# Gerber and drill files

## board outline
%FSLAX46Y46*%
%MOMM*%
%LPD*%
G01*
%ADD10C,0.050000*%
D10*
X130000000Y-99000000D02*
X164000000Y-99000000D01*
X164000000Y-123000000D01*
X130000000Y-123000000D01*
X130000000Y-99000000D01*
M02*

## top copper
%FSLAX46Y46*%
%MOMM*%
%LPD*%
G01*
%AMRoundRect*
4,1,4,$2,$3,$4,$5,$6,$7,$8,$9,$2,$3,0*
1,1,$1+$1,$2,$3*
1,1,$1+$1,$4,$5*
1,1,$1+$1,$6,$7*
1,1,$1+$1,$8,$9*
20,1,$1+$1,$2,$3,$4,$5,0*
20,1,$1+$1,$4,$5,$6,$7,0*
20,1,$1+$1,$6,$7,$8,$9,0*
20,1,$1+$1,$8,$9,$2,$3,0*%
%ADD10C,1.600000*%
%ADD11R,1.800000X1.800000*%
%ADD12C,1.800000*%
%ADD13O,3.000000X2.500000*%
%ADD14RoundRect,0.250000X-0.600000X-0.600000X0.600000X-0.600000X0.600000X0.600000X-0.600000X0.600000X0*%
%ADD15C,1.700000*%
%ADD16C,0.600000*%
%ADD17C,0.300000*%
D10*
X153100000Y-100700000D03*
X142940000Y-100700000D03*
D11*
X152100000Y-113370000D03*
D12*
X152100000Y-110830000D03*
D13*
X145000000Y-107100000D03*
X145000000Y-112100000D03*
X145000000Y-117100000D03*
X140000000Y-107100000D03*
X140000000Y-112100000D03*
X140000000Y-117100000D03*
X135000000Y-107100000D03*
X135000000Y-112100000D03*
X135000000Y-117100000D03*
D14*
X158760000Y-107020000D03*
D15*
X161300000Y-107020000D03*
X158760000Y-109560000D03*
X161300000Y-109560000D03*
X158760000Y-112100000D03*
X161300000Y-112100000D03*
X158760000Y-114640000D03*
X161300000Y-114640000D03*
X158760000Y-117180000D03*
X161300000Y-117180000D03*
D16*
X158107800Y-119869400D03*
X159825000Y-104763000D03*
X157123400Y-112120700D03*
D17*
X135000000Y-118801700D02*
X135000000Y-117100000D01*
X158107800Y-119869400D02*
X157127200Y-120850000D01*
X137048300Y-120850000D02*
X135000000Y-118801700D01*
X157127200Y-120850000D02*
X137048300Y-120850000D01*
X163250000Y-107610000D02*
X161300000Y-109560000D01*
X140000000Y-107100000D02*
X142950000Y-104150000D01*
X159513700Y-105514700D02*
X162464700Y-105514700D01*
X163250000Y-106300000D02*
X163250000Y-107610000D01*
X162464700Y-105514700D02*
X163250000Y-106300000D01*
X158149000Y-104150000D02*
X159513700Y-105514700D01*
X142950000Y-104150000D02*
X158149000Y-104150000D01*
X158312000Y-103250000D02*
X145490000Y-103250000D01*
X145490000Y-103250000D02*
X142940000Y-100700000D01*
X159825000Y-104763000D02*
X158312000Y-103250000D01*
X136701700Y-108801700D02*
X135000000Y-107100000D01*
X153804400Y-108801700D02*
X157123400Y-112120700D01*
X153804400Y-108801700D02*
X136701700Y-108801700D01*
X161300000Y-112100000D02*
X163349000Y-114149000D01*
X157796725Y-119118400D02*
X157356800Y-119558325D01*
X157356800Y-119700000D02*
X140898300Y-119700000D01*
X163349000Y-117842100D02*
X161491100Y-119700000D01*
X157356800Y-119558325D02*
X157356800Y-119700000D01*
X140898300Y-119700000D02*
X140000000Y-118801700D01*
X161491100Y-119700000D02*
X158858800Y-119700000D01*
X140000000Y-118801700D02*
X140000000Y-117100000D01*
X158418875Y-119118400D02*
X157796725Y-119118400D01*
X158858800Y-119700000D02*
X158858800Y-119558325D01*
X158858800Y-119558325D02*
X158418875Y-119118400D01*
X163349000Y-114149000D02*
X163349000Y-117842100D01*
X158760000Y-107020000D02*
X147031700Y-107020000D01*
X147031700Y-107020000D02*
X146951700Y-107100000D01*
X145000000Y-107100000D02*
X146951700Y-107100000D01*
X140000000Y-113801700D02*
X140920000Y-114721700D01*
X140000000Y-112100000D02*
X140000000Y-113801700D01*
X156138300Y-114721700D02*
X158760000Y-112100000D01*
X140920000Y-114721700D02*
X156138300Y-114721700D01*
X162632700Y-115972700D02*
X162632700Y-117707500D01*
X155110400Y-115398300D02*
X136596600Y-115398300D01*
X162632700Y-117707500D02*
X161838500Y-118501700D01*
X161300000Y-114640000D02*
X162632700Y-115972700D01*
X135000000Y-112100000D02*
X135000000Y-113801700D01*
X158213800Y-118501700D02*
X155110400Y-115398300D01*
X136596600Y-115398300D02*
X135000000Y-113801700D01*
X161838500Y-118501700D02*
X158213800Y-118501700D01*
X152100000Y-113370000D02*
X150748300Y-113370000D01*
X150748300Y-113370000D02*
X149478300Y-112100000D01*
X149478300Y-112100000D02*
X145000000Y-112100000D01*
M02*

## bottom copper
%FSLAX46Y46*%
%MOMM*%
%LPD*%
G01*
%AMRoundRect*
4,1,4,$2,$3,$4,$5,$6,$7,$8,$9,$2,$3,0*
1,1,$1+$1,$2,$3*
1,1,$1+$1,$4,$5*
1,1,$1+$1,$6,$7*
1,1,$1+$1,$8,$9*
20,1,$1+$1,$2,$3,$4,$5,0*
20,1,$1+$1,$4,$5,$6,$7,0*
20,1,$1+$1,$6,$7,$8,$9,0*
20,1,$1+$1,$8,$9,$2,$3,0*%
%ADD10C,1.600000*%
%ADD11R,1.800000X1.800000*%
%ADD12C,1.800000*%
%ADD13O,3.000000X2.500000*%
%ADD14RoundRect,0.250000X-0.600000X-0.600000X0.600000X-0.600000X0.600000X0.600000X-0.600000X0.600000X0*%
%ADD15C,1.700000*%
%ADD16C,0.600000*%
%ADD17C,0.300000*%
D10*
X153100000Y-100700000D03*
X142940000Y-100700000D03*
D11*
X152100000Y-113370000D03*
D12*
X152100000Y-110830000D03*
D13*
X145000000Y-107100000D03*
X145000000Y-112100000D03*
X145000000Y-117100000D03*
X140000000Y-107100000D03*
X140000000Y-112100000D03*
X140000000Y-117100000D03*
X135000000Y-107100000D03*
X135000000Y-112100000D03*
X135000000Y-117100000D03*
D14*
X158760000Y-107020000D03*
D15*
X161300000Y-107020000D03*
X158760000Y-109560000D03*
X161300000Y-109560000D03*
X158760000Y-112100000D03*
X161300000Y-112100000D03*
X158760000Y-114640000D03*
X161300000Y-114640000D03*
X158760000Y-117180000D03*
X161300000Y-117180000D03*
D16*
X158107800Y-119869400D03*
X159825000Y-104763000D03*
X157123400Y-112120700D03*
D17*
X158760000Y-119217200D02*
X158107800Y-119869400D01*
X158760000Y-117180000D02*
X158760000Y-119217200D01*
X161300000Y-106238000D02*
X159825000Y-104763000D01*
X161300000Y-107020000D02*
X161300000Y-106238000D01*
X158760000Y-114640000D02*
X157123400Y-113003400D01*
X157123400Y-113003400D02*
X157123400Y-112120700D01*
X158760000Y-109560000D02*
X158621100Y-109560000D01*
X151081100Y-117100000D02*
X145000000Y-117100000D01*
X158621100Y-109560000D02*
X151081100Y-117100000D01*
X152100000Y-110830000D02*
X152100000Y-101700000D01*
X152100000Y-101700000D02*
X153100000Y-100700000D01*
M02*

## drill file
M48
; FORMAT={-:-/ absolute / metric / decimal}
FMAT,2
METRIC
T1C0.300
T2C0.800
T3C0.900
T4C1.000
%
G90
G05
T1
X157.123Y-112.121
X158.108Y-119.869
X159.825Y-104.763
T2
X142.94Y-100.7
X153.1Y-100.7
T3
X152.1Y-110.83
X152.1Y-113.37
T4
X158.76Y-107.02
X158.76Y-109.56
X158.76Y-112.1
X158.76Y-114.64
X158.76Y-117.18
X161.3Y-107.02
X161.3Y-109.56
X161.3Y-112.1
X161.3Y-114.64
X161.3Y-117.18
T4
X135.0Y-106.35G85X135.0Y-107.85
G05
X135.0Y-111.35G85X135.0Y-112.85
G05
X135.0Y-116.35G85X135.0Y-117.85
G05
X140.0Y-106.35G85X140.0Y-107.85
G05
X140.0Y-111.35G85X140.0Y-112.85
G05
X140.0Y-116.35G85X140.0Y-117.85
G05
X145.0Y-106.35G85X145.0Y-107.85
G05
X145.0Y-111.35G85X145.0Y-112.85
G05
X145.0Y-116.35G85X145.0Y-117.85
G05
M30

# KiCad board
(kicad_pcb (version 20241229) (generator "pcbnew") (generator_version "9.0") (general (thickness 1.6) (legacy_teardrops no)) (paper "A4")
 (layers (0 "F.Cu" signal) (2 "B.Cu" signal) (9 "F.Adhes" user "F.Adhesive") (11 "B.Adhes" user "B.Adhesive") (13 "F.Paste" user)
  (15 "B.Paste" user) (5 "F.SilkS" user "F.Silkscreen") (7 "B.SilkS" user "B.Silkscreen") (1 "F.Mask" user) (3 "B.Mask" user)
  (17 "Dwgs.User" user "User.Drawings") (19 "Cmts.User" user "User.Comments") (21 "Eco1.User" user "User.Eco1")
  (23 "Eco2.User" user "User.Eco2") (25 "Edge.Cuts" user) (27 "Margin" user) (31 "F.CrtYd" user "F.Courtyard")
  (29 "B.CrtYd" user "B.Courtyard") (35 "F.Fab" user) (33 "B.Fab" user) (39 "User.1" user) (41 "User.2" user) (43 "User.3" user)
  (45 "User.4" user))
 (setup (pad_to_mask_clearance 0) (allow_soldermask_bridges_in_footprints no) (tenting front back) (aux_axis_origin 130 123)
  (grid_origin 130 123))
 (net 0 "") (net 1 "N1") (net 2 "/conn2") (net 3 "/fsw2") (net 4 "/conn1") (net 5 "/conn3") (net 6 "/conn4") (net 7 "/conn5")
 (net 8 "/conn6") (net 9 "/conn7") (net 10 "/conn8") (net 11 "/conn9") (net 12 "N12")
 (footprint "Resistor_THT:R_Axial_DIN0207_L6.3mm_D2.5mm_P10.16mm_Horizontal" (layer "F.Cu") (at 153.1 100.7 180)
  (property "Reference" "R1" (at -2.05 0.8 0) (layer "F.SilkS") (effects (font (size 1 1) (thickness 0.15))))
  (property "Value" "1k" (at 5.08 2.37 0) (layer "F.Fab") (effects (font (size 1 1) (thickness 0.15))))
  (pad "1" thru_hole circle (at 0 0 180) (size 1.6 1.6) (drill 0.8) (layers "*.Cu" "*.Mask") (remove_unused_layers no) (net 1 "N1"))
  (pad "2" thru_hole circle (at 10.16 0 180) (size 1.6 1.6) (drill 0.8) (layers "*.Cu" "*.Mask") (remove_unused_layers no) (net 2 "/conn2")))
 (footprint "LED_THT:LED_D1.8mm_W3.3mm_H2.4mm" (layer "F.Cu") (at 152.1 113.37 90)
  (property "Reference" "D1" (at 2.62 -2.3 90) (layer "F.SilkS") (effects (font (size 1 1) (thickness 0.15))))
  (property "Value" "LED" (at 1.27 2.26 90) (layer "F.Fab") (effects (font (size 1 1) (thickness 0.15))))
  (pad "1" thru_hole rect (at 0 0 90) (size 1.8 1.8) (drill 0.9) (layers "*.Cu" "*.Mask") (remove_unused_layers no) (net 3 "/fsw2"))
  (pad "2" thru_hole circle (at 2.54 0 90) (size 1.8 1.8) (drill 0.9) (layers "*.Cu" "*.Mask") (remove_unused_layers no) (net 1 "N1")))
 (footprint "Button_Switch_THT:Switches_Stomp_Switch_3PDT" (layer "F.Cu") (at 140 112.1 -90)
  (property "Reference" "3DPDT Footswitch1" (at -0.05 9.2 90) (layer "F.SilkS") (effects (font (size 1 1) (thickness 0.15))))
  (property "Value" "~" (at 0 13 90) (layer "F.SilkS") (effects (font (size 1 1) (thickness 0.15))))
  (pad "1" thru_hole oval (at -5 -5 270) (size 2.5 3) (drill oval 2.5 1) (layers "*.Cu" "*.Mask" "F.SilkS") (remove_unused_layers no)
   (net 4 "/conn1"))
  (pad "2" thru_hole oval (at 0 -5 270) (size 2.5 3) (drill oval 2.5 1) (layers "*.Cu" "*.Mask" "F.SilkS") (remove_unused_layers no)
   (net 3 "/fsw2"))
  (pad "3" thru_hole oval (at 5 -5 270) (size 2.5 3) (drill oval 2.5 1) (layers "*.Cu" "*.Mask" "F.SilkS") (remove_unused_layers no)
   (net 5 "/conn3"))
  (pad "4" thru_hole oval (at -5 0 270) (size 2.5 3) (drill oval 2.5 1) (layers "*.Cu" "*.Mask" "F.SilkS") (remove_unused_layers no)
   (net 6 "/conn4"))
  (pad "5" thru_hole oval (at 0 0 270) (size 2.5 3) (drill oval 2.5 1) (layers "*.Cu" "*.Mask" "F.SilkS") (remove_unused_layers no)
   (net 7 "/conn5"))
  (pad "6" thru_hole oval (at 5 0 270) (size 2.5 3) (drill oval 2.5 1) (layers "*.Cu" "*.Mask" "F.SilkS") (remove_unused_layers no)
   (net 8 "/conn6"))
  (pad "7" thru_hole oval (at -5 5 270) (size 2.5 3) (drill oval 2.5 1) (layers "*.Cu" "*.Mask" "F.SilkS") (remove_unused_layers no)
   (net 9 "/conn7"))
  (pad "8" thru_hole oval (at 0 5 270) (size 2.5 3) (drill oval 2.5 1) (layers "*.Cu" "*.Mask" "F.SilkS") (remove_unused_layers no)
   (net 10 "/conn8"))
  (pad "9" thru_hole oval (at 5 5 270) (size 2.5 3) (drill oval 2.5 1) (layers "*.Cu" "*.Mask" "F.SilkS") (remove_unused_layers no)
   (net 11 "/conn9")))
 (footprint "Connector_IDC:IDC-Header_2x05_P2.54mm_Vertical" (layer "F.Cu") (at 158.76 107.02)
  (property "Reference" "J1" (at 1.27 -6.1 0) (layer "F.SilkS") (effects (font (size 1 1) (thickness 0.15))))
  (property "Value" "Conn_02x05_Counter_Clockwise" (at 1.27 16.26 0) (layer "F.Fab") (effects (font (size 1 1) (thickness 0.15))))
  (pad "1" thru_hole roundrect (at 0 0) (size 1.7 1.7) (drill 1) (layers "*.Cu" "*.Mask") (remove_unused_layers no)
   (roundrect_rratio 0.147059) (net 4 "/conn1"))
  (pad "2" thru_hole circle (at 2.54 0) (size 1.7 1.7) (drill 1) (layers "*.Cu" "*.Mask") (remove_unused_layers no) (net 2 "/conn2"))
  (pad "3" thru_hole circle (at 0 2.54) (size 1.7 1.7) (drill 1) (layers "*.Cu" "*.Mask") (remove_unused_layers no) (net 5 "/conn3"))
  (pad "4" thru_hole circle (at 2.54 2.54) (size 1.7 1.7) (drill 1) (layers "*.Cu" "*.Mask") (remove_unused_layers no) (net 6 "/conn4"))
  (pad "5" thru_hole circle (at 0 5.08) (size 1.7 1.7) (drill 1) (layers "*.Cu" "*.Mask") (remove_unused_layers no) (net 7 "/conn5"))
  (pad "6" thru_hole circle (at 2.54 5.08) (size 1.7 1.7) (drill 1) (layers "*.Cu" "*.Mask") (remove_unused_layers no) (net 8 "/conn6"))
  (pad "7" thru_hole circle (at 0 7.62) (size 1.7 1.7) (drill 1) (layers "*.Cu" "*.Mask") (remove_unused_layers no) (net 9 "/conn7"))
  (pad "8" thru_hole circle (at 2.54 7.62) (size 1.7 1.7) (drill 1) (layers "*.Cu" "*.Mask") (remove_unused_layers no) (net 10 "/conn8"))
  (pad "9" thru_hole circle (at 0 10.16) (size 1.7 1.7) (drill 1) (layers "*.Cu" "*.Mask") (remove_unused_layers no) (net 11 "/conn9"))
  (pad "10" thru_hole circle (at 2.54 10.16) (size 1.7 1.7) (drill 1) (layers "*.Cu" "*.Mask") (remove_unused_layers no) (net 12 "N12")))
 (gr_rect (start 130 99) (end 164 123) (stroke (width 0.05) (type solid)) (fill no) (layer "Edge.Cuts"))
 (segment (start 135 118.8017) (end 135 117.1) (width 0.3) (layer "F.Cu") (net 11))
 (segment (start 158.1078 119.8694) (end 157.1272 120.85) (width 0.3) (layer "F.Cu") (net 11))
 (segment (start 137.0483 120.85) (end 135 118.8017) (width 0.3) (layer "F.Cu") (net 11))
 (segment (start 157.1272 120.85) (end 137.0483 120.85) (width 0.3) (layer "F.Cu") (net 11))
 (via (at 158.1078 119.8694) (size 0.6) (drill 0.3) (layers "F.Cu" "B.Cu") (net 11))
 (segment (start 158.76 119.2172) (end 158.1078 119.8694) (width 0.3) (layer "B.Cu") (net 11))
 (segment (start 158.76 117.18) (end 158.76 119.2172) (width 0.3) (layer "B.Cu") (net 11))
 (segment (start 163.25 107.61) (end 161.3 109.56) (width 0.3) (layer "F.Cu") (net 6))
 (segment (start 140 107.1) (end 142.95 104.15) (width 0.3) (layer "F.Cu") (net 6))
 (segment (start 159.5137 105.5147) (end 162.4647 105.5147) (width 0.3) (layer "F.Cu") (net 6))
 (segment (start 163.25 106.3) (end 163.25 107.61) (width 0.3) (layer "F.Cu") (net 6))
 (segment (start 162.4647 105.5147) (end 163.25 106.3) (width 0.3) (layer "F.Cu") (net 6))
 (segment (start 158.149 104.15) (end 159.5137 105.5147) (width 0.3) (layer "F.Cu") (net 6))
 (segment (start 142.95 104.15) (end 158.149 104.15) (width 0.3) (layer "F.Cu") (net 6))
 (segment (start 158.312 103.25) (end 145.49 103.25) (width 0.3) (layer "F.Cu") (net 2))
 (segment (start 145.49 103.25) (end 142.94 100.7) (width 0.3) (layer "F.Cu") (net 2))
 (segment (start 159.825 104.763) (end 158.312 103.25) (width 0.3) (layer "F.Cu") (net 2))
 (via (at 159.825 104.763) (size 0.6) (drill 0.3) (layers "F.Cu" "B.Cu") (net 2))
 (segment (start 161.3 106.238) (end 159.825 104.763) (width 0.3) (layer "B.Cu") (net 2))
 (segment (start 161.3 107.02) (end 161.3 106.238) (width 0.3) (layer "B.Cu") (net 2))
 (segment (start 136.7017 108.8017) (end 135 107.1) (width 0.3) (layer "F.Cu") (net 9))
 (segment (start 153.8044 108.8017) (end 157.1234 112.1207) (width 0.3) (layer "F.Cu") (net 9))
 (segment (start 153.8044 108.8017) (end 136.7017 108.8017) (width 0.3) (layer "F.Cu") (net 9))
 (via (at 157.1234 112.1207) (size 0.6) (drill 0.3) (layers "F.Cu" "B.Cu") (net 9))
 (segment (start 158.76 114.64) (end 157.1234 113.0034) (width 0.3) (layer "B.Cu") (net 9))
 (segment (start 157.1234 113.0034) (end 157.1234 112.1207) (width 0.3) (layer "B.Cu") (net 9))
 (segment (start 158.76 109.56) (end 158.6211 109.56) (width 0.3) (layer "B.Cu") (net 5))
 (segment (start 151.0811 117.1) (end 145 117.1) (width 0.3) (layer "B.Cu") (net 5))
 (segment (start 158.6211 109.56) (end 151.0811 117.1) (width 0.3) (layer "B.Cu") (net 5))
 (segment (start 161.3 112.1) (end 163.349 114.149) (width 0.3) (layer "F.Cu") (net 8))
 (segment (start 157.796725 119.1184) (end 157.3568 119.558325) (width 0.3) (layer "F.Cu") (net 8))
 (segment (start 157.3568 119.7) (end 140.8983 119.7) (width 0.3) (layer "F.Cu") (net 8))
 (segment (start 163.349 117.8421) (end 161.4911 119.7) (width 0.3) (layer "F.Cu") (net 8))
 (segment (start 157.3568 119.558325) (end 157.3568 119.7) (width 0.3) (layer "F.Cu") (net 8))
 (segment (start 140.8983 119.7) (end 140 118.8017) (width 0.3) (layer "F.Cu") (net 8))
 (segment (start 161.4911 119.7) (end 158.8588 119.7) (width 0.3) (layer "F.Cu") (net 8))
 (segment (start 140 118.8017) (end 140 117.1) (width 0.3) (layer "F.Cu") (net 8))
 (segment (start 158.418875 119.1184) (end 157.796725 119.1184) (width 0.3) (layer "F.Cu") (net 8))
 (segment (start 158.8588 119.7) (end 158.8588 119.558325) (width 0.3) (layer "F.Cu") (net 8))
 (segment (start 158.8588 119.558325) (end 158.418875 119.1184) (width 0.3) (layer "F.Cu") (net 8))
 (segment (start 163.349 114.149) (end 163.349 117.8421) (width 0.3) (layer "F.Cu") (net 8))
 (segment (start 158.76 107.02) (end 147.0317 107.02) (width 0.3) (layer "F.Cu") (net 4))
 (segment (start 147.0317 107.02) (end 146.9517 107.1) (width 0.3) (layer "F.Cu") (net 4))
 (segment (start 145 107.1) (end 146.9517 107.1) (width 0.3) (layer "F.Cu") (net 4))
 (segment (start 140 113.8017) (end 140.92 114.7217) (width 0.3) (layer "F.Cu") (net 7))
 (segment (start 140 112.1) (end 140 113.8017) (width 0.3) (layer "F.Cu") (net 7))
 (segment (start 156.1383 114.7217) (end 158.76 112.1) (width 0.3) (layer "F.Cu") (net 7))
 (segment (start 140.92 114.7217) (end 156.1383 114.7217) (width 0.3) (layer "F.Cu") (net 7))
 (segment (start 162.6327 115.9727) (end 162.6327 117.7075) (width 0.3) (layer "F.Cu") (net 10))
 (segment (start 155.1104 115.3983) (end 136.5966 115.3983) (width 0.3) (layer "F.Cu") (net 10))
 (segment (start 162.6327 117.7075) (end 161.8385 118.5017) (width 0.3) (layer "F.Cu") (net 10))
 (segment (start 161.3 114.64) (end 162.6327 115.9727) (width 0.3) (layer "F.Cu") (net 10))
 (segment (start 135 112.1) (end 135 113.8017) (width 0.3) (layer "F.Cu") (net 10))
 (segment (start 158.2138 118.5017) (end 155.1104 115.3983) (width 0.3) (layer "F.Cu") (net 10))
 (segment (start 136.5966 115.3983) (end 135 113.8017) (width 0.3) (layer "F.Cu") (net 10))
 (segment (start 161.8385 118.5017) (end 158.2138 118.5017) (width 0.3) (layer "F.Cu") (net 10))
 (segment (start 152.1 110.83) (end 152.1 101.7) (width 0.3) (layer "B.Cu") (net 1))
 (segment (start 152.1 101.7) (end 153.1 100.7) (width 0.3) (layer "B.Cu") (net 1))
 (segment (start 152.1 113.37) (end 150.7483 113.37) (width 0.3) (layer "F.Cu") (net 3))
 (segment (start 150.7483 113.37) (end 149.4783 112.1) (width 0.3) (layer "F.Cu") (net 3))
 (segment (start 149.4783 112.1) (end 145 112.1) (width 0.3) (layer "F.Cu") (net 3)))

